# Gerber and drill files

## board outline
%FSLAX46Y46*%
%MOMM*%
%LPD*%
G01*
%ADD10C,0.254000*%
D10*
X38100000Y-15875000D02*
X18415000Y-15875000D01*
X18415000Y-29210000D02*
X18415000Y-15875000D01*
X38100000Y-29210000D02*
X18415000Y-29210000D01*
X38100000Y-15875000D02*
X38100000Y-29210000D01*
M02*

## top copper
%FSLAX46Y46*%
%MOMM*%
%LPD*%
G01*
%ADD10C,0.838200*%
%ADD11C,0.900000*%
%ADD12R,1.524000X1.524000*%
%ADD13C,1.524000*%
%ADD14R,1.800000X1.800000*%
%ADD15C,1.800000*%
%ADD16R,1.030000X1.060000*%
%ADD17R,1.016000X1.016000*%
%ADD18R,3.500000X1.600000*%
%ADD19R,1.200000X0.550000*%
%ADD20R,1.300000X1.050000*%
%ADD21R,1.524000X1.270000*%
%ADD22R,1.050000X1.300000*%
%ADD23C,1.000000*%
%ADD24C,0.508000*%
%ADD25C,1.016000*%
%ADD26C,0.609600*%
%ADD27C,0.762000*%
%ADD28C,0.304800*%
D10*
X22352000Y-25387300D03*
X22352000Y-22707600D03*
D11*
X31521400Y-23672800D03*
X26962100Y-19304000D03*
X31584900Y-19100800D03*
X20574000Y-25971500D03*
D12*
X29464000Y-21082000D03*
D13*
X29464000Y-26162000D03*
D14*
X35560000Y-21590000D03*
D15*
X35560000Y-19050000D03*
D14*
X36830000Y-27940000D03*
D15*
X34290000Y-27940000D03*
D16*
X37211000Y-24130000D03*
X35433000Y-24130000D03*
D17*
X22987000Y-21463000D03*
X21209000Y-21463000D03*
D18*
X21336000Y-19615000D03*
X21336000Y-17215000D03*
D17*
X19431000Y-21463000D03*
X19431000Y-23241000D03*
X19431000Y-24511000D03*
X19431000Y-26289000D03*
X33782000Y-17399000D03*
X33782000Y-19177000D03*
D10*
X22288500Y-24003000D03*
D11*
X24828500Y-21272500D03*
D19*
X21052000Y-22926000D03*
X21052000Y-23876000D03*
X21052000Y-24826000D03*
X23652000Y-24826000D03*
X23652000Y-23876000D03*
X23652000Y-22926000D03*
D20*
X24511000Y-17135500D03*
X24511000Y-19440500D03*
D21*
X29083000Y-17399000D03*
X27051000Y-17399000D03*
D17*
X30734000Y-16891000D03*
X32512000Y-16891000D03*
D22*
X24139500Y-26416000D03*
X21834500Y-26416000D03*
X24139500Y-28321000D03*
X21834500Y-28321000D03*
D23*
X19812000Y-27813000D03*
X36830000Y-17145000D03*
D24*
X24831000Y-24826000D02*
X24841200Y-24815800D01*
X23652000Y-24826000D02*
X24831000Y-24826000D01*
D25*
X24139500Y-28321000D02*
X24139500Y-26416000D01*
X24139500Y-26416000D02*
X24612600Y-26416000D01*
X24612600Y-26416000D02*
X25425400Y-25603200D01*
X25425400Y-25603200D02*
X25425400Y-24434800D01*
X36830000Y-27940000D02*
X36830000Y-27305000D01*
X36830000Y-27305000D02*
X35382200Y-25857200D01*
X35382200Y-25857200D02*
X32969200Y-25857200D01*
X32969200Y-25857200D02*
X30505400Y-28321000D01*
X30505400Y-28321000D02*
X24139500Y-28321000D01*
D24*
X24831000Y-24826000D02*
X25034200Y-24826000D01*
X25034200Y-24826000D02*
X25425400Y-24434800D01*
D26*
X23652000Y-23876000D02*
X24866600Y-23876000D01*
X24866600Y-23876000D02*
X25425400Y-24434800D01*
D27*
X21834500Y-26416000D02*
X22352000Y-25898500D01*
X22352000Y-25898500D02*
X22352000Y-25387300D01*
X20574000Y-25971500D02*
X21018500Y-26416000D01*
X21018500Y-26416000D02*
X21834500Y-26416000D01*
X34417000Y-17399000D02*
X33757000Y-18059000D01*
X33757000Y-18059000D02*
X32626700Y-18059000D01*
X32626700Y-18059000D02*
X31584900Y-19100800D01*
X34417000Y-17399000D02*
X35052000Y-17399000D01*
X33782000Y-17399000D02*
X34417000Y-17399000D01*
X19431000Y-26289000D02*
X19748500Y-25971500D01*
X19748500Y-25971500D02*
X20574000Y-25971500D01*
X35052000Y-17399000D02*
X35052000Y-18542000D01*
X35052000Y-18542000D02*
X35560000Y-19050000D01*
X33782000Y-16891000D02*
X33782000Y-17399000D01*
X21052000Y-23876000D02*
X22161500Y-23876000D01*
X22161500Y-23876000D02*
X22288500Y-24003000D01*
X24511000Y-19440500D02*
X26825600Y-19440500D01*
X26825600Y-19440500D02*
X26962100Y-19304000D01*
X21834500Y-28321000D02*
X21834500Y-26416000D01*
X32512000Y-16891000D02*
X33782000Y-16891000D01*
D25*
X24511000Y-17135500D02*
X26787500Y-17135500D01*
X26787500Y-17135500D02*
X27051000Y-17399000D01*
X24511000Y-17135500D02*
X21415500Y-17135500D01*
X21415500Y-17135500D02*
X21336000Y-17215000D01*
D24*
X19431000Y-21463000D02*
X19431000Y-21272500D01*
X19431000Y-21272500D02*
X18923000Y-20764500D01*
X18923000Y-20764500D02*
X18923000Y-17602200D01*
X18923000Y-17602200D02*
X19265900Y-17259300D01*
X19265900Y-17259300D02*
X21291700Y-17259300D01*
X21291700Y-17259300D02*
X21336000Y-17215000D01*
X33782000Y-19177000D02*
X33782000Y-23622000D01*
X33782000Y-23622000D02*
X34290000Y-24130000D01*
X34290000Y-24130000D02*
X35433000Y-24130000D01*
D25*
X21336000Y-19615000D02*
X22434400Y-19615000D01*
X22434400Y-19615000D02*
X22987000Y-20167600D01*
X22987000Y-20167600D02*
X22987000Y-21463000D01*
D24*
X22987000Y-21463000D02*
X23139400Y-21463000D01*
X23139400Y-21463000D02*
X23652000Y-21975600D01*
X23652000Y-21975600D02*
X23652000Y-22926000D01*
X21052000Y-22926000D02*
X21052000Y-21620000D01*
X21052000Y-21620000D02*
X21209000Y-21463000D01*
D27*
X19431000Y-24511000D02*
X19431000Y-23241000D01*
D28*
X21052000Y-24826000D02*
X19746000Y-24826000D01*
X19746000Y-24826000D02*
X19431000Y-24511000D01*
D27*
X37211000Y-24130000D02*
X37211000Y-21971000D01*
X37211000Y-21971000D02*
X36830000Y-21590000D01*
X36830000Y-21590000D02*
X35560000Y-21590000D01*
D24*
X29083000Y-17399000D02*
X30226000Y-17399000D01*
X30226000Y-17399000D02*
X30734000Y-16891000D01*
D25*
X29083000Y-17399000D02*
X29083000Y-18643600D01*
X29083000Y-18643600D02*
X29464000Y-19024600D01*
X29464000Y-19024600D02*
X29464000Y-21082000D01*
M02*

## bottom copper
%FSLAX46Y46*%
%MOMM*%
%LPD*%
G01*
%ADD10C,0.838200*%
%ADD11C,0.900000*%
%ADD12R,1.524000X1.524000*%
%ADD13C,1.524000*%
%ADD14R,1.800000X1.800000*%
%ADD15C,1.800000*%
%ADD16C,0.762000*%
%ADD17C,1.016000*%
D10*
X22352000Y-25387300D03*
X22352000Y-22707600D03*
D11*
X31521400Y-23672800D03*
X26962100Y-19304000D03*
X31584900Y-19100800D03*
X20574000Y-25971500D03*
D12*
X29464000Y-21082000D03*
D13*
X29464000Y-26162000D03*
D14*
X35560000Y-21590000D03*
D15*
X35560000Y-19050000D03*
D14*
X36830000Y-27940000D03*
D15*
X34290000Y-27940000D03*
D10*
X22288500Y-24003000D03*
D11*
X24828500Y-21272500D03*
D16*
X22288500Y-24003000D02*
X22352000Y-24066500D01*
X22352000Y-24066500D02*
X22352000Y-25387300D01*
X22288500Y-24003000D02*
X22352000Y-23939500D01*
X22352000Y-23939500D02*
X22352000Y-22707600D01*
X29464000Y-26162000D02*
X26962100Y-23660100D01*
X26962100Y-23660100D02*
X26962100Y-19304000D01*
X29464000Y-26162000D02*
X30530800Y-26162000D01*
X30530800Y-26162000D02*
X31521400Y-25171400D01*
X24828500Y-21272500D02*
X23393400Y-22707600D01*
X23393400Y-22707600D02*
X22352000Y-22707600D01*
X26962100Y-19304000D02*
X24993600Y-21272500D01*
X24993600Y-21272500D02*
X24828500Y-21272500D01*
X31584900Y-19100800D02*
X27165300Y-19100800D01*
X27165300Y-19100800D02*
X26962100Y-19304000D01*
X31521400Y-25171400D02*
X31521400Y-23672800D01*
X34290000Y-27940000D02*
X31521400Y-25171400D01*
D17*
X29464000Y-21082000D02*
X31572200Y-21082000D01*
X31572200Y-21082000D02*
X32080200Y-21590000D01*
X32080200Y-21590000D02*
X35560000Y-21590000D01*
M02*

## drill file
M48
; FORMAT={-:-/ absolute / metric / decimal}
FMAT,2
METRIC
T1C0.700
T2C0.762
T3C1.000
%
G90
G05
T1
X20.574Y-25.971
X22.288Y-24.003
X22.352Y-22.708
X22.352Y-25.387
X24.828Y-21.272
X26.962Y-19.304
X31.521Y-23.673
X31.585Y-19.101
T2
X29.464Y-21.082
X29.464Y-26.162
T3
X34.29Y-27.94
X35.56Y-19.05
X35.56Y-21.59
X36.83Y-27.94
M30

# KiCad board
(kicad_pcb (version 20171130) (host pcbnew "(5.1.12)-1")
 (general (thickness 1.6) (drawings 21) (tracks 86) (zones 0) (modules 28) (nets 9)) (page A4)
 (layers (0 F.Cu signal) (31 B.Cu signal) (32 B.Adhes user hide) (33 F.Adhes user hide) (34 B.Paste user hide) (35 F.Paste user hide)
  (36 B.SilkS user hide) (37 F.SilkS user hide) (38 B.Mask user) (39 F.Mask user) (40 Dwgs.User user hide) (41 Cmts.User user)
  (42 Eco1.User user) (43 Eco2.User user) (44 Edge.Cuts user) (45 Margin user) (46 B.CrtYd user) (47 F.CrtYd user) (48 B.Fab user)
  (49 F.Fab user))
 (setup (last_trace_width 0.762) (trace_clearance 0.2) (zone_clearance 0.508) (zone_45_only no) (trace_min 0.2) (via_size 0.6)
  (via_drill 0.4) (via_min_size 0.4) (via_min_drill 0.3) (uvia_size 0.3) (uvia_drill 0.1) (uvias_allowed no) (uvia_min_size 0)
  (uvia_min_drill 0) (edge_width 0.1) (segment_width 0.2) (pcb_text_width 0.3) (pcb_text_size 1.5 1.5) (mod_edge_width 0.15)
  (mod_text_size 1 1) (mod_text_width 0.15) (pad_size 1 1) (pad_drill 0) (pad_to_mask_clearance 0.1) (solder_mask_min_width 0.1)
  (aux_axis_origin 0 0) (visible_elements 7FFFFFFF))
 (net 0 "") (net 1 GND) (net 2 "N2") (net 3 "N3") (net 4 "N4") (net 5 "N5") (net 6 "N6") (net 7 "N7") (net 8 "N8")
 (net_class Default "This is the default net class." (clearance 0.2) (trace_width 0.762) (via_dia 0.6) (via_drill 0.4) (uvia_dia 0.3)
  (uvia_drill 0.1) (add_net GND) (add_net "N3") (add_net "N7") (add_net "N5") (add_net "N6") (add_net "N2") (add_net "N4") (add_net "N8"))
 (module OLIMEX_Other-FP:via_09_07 (layer F.Cu) (at 22.352 25.3873)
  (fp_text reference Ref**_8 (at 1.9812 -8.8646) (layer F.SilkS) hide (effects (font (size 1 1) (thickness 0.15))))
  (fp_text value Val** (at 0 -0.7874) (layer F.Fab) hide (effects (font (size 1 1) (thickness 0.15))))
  (pad 0 thru_hole circle (at 0 0) (size 0.8382 0.8382) (drill 0.7) (layers *.Cu) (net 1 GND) (zone_connect 2)))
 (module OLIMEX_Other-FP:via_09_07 (layer F.Cu) (at 22.352 22.7076)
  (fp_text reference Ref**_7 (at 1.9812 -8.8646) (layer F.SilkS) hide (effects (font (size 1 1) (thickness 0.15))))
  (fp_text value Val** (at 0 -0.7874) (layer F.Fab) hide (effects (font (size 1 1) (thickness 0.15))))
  (pad 0 thru_hole circle (at 0 0) (size 0.8382 0.8382) (drill 0.7) (layers *.Cu) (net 1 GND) (zone_connect 2)))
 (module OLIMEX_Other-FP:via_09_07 (layer F.Cu) (at 31.5214 23.7363)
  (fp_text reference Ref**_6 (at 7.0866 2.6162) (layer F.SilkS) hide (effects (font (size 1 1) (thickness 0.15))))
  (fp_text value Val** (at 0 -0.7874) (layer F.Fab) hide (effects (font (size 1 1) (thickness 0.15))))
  (pad 0 thru_hole circle (at 0 -0.0635) (size 0.9 0.9) (drill 0.7) (layers *.Cu) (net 1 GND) (zone_connect 2)))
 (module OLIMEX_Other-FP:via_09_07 (layer F.Cu) (at 26.9621 19.3675)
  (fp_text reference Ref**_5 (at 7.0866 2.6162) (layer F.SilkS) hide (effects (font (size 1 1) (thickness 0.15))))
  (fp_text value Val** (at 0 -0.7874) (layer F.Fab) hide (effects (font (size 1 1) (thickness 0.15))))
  (pad 0 thru_hole circle (at 0 -0.0635) (size 0.9 0.9) (drill 0.7) (layers *.Cu) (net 1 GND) (zone_connect 2)))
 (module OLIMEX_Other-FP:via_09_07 (layer F.Cu) (at 31.5849 19.1643)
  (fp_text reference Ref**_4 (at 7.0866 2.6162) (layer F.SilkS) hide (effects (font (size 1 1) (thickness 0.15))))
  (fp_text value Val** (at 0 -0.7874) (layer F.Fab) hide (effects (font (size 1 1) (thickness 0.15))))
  (pad 0 thru_hole circle (at 0 -0.0635) (size 0.9 0.9) (drill 0.7) (layers *.Cu) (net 1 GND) (zone_connect 2)))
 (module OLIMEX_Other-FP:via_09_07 (layer F.Cu) (at 20.574 26.035)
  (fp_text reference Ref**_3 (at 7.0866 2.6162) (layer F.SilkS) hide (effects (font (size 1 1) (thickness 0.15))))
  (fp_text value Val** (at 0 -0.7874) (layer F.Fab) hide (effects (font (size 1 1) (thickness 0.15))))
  (pad 0 thru_hole circle (at 0 -0.0635) (size 0.9 0.9) (drill 0.7) (layers *.Cu) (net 1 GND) (zone_connect 2)))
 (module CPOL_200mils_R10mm (layer F.Cu) (at 29.464 23.622 270)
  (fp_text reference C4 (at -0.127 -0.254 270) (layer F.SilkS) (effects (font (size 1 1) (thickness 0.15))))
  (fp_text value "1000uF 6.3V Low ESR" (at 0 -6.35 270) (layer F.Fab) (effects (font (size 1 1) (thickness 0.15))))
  (pad 1 thru_hole rect (at -2.54 0 270) (size 1.524 1.524) (drill 0.762) (layers *.Cu *.Mask F.SilkS) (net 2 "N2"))
  (pad 2 thru_hole circle (at 2.54 0 270) (size 1.524 1.524) (drill 0.762) (layers *.Cu *.Mask F.SilkS) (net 1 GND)))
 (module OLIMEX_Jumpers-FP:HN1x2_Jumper (layer F.Cu) (at 35.56 20.32 90)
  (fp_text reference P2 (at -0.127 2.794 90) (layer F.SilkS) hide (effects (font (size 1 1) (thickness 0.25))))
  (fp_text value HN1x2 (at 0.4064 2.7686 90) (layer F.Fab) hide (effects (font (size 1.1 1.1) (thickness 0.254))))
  (pad 1 thru_hole rect (at -1.27 0 180) (size 1.8 1.8) (drill 1) (layers *.Cu *.Mask F.SilkS) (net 2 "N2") (solder_mask_margin 0.0508)
   (solder_paste_margin -0.0508))
  (pad 2 thru_hole circle (at 1.27 0 180) (size 1.8 1.8) (drill 1) (layers *.Cu *.Mask F.SilkS) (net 1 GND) (solder_mask_margin 0.0508)
   (solder_paste_margin -0.0508)))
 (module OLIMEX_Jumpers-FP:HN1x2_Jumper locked (layer F.Cu) (at 35.56 27.94 180)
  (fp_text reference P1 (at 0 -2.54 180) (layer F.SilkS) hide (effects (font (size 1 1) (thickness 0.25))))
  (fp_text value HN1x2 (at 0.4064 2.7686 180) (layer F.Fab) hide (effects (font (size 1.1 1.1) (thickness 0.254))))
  (pad 1 thru_hole rect (at -1.27 0 270) (size 1.8 1.8) (drill 1) (layers *.Cu *.Mask F.SilkS) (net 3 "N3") (solder_mask_margin 0.0508)
   (solder_paste_margin -0.0508))
  (pad 2 thru_hole circle (at 1.27 0 270) (size 1.8 1.8) (drill 1) (layers *.Cu *.Mask F.SilkS) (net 1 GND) (solder_mask_margin 0.0508)
   (solder_paste_margin -0.0508)))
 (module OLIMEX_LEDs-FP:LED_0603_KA (layer F.Cu) (at 36.322 24.13 180)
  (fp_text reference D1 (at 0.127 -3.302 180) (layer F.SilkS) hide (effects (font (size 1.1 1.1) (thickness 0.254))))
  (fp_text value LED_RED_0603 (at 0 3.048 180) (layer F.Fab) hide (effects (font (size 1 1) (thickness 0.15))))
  (pad 2 smd rect (at -0.889 0 180) (size 1.03 1.06) (layers F.Cu F.Paste F.Mask) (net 2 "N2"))
  (pad 1 smd rect (at 0.889 0 180) (size 1.03 1.06) (layers F.Cu F.Paste F.Mask) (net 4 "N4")))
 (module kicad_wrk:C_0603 (layer F.Cu) (at 22.098 21.463 180)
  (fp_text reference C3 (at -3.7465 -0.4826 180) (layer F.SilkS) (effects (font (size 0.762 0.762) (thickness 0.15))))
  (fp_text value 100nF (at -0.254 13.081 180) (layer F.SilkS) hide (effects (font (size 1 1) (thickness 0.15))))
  (pad 1 smd rect (at -0.889 0 180) (size 1.016 1.016) (layers F.Cu F.Paste F.Mask) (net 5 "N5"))
  (pad 2 smd rect (at 0.889 0 180) (size 1.016 1.016) (layers F.Cu F.Paste F.Mask) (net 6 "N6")))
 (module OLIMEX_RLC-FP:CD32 (layer F.Cu) (at 21.336 18.415 90)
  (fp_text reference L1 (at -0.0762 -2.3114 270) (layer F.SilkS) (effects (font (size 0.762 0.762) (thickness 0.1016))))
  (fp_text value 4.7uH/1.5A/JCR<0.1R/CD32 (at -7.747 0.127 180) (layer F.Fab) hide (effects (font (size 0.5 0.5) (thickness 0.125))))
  (pad 1 smd rect (at -1.2 0 180) (size 3.5 1.6) (layers F.Cu F.Paste F.Mask) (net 5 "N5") (solder_mask_margin 0.0508)
   (solder_paste_margin -0.0508) (clearance 0.0508))
  (pad 2 smd rect (at 1.2 0 180) (size 3.5 1.6) (layers F.Cu F.Paste F.Mask) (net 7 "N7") (solder_mask_margin 0.0508)
   (solder_paste_margin -0.0508) (clearance 0.0508)))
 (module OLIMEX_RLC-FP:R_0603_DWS (layer F.Cu) (at 19.431 22.352 270)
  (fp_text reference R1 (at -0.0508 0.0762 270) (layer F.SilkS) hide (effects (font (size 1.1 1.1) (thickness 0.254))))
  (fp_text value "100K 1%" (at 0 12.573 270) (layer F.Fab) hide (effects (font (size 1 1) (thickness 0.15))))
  (pad 1 smd rect (at -0.889 0 270) (size 1.016 1.016) (layers F.Cu F.Paste F.Mask) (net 7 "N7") (solder_mask_margin 0.0508)
   (solder_paste_margin -0.0508) (clearance 0.0508))
  (pad 2 smd rect (at 0.889 0 270) (size 1.016 1.016) (layers F.Cu F.Paste F.Mask) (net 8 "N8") (solder_mask_margin 0.0508)
   (solder_paste_margin -0.0508) (clearance 0.0508)))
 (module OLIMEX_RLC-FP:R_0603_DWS (layer F.Cu) (at 19.431 25.4 270)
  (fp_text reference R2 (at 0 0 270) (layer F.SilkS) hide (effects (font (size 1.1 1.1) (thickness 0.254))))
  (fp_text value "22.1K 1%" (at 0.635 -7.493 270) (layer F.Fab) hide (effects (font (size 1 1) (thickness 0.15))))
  (pad 1 smd rect (at -0.889 0 270) (size 1.016 1.016) (layers F.Cu F.Paste F.Mask) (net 8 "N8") (solder_mask_margin 0.0508)
   (solder_paste_margin -0.0508) (clearance 0.0508))
  (pad 2 smd rect (at 0.889 0 270) (size 1.016 1.016) (layers F.Cu F.Paste F.Mask) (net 1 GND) (solder_mask_margin 0.0508)
   (solder_paste_margin -0.0508) (clearance 0.0508)))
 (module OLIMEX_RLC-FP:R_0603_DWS (layer F.Cu) (at 33.782 18.288 270)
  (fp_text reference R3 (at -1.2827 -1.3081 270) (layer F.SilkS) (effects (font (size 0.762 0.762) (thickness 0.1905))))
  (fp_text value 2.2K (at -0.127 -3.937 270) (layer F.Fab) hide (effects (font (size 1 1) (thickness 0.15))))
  (pad 1 smd rect (at -0.889 0 270) (size 1.016 1.016) (layers F.Cu F.Paste F.Mask) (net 1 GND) (solder_mask_margin 0.0508)
   (solder_paste_margin -0.0508) (clearance 0.0508))
  (pad 2 smd rect (at 0.889 0 270) (size 1.016 1.016) (layers F.Cu F.Paste F.Mask) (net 4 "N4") (solder_mask_margin 0.0508)
   (solder_paste_margin -0.0508) (clearance 0.0508)))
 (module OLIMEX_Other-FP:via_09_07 (layer F.Cu) (at 22.2885 24.003)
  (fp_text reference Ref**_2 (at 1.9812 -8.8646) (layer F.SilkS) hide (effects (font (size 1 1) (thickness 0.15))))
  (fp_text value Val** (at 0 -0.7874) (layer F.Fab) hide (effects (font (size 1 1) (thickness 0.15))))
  (pad 0 thru_hole circle (at 0 0) (size 0.8382 0.8382) (drill 0.7) (layers *.Cu) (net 1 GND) (zone_connect 2)))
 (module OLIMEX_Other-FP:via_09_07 (layer F.Cu) (at 24.8285 21.336)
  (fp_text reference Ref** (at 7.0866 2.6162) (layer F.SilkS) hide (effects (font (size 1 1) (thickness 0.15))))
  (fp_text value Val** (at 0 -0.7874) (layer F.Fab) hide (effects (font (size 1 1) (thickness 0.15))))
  (pad 0 thru_hole circle (at 0 -0.0635) (size 0.9 0.9) (drill 0.7) (layers *.Cu) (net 1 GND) (zone_connect 2)))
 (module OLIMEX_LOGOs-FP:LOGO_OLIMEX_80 (layer B.Cu) (at 27.6606 23.0378 180)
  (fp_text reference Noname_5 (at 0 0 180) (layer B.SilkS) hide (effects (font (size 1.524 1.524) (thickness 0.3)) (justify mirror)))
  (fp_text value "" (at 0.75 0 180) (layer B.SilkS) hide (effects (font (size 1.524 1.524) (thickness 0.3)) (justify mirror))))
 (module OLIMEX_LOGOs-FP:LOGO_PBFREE (layer B.Cu) (at 26.5938 18.796 180)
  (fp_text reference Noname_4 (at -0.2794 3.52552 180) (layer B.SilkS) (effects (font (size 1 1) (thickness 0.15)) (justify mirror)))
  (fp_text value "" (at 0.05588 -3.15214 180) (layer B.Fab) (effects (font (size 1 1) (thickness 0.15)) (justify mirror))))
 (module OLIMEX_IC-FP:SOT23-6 (layer F.Cu) (at 22.352 23.876 180)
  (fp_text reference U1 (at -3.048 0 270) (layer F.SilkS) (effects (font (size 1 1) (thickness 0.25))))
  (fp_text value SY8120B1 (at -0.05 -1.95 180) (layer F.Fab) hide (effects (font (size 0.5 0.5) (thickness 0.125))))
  (pad 1 smd rect (at 1.3 0.95 270) (size 0.55 1.2) (layers F.Cu F.Paste F.Mask) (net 6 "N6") (solder_mask_margin 0.0508)
   (solder_paste_margin -0.0508) (clearance 0.0508))
  (pad 2 smd rect (at 1.3 0 270) (size 0.55 1.2) (layers F.Cu F.Paste F.Mask) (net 1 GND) (solder_mask_margin 0.0508)
   (solder_paste_margin -0.0508) (clearance 0.0508))
  (pad 3 smd rect (at 1.3 -0.95 270) (size 0.55 1.2) (layers F.Cu F.Paste F.Mask) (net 8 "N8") (solder_mask_margin 0.0508)
   (solder_paste_margin -0.0508) (clearance 0.0508))
  (pad 4 smd rect (at -1.3 -0.95 270) (size 0.55 1.2) (layers F.Cu F.Paste F.Mask) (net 3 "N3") (solder_mask_margin 0.0508)
   (solder_paste_margin -0.0508) (clearance 0.0508))
  (pad 5 smd rect (at -1.3 0 270) (size 0.55 1.2) (layers F.Cu F.Paste F.Mask) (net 3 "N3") (solder_mask_margin 0.0508)
   (solder_paste_margin -0.0508) (clearance 0.0508))
  (pad 6 smd rect (at -1.3 0.95 270) (size 0.55 1.2) (layers F.Cu F.Paste F.Mask) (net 5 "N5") (solder_mask_margin 0.0508)
   (solder_paste_margin -0.0508) (clearance 0.0508)))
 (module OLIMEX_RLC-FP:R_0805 (layer F.Cu) (at 24.511 18.288)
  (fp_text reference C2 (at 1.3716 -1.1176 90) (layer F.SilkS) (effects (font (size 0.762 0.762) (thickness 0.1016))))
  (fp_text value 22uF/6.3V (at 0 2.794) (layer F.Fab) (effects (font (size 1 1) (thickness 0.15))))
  (pad 1 smd rect (at 0 -1.1525) (size 1.3 1.05) (layers F.Cu F.Paste F.Mask) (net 7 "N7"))
  (pad 2 smd rect (at 0 1.1525) (size 1.3 1.05) (layers F.Cu F.Paste F.Mask) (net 1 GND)))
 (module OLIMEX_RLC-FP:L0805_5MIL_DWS (layer F.Cu) (at 28.067 17.399)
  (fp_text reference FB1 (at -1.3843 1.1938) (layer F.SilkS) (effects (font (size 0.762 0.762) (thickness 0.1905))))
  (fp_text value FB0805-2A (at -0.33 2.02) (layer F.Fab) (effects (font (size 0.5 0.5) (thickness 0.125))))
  (pad 2 smd rect (at 1.016 0) (size 1.524 1.27) (layers F.Cu F.Paste F.Mask) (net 2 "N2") (solder_mask_margin 0.0508)
   (solder_paste_margin -0.0508) (clearance 0.0508))
  (pad 1 smd rect (at -1.016 0) (size 1.524 1.27) (layers F.Cu F.Paste F.Mask) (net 7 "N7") (solder_mask_margin 0.0508)
   (solder_paste_margin -0.0508) (clearance 0.0508)))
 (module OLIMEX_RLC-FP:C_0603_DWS (layer F.Cu) (at 31.623 16.891)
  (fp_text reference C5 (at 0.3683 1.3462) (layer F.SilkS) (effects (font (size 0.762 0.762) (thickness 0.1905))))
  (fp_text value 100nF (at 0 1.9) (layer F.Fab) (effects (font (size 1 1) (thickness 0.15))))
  (pad 1 smd rect (at -0.889 0) (size 1.016 1.016) (layers F.Cu F.Paste F.Mask) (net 2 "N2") (solder_mask_margin 0.0508)
   (solder_paste_margin -0.0508) (clearance 0.0508))
  (pad 2 smd rect (at 0.889 0) (size 1.016 1.016) (layers F.Cu F.Paste F.Mask) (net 1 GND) (solder_mask_margin 0.0508)
   (solder_paste_margin -0.0508) (clearance 0.0508)))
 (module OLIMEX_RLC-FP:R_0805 (layer F.Cu) (at 22.987 26.416 270)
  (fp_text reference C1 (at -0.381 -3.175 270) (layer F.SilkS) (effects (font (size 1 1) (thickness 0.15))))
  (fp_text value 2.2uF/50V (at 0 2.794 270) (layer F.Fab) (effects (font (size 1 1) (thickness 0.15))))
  (pad 1 smd rect (at 0 -1.1525 270) (size 1.3 1.05) (layers F.Cu F.Paste F.Mask) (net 3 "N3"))
  (pad 2 smd rect (at 0 1.1525 270) (size 1.3 1.05) (layers F.Cu F.Paste F.Mask) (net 1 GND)))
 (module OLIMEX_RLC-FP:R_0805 (layer F.Cu) (at 22.987 28.321 270)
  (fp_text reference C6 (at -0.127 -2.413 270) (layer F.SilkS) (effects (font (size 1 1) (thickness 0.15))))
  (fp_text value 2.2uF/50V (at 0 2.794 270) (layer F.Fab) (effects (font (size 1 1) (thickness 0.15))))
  (pad 1 smd rect (at 0 -1.1525 270) (size 1.3 1.05) (layers F.Cu F.Paste F.Mask) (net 3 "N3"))
  (pad 2 smd rect (at 0 1.1525 270) (size 1.3 1.05) (layers F.Cu F.Paste F.Mask) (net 1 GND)))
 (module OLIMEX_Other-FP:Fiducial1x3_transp (layer F.Cu) (at 19.812 27.813)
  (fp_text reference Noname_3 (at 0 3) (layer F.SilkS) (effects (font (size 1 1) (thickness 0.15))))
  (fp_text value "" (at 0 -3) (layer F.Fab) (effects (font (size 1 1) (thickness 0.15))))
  (pad Fid1 connect circle (at 0 0) (size 1 1) (layers F.Cu F.Mask) (clearance 0.4) (zone_connect 0)))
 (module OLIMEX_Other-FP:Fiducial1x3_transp (layer F.Cu) (at 36.83 17.145)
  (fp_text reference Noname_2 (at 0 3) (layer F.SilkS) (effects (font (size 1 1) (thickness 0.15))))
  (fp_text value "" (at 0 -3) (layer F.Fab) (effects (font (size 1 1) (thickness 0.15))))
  (pad Fid1 connect circle (at 0 0) (size 1 1) (layers F.Cu F.Mask) (clearance 0.6) (zone_connect 0)))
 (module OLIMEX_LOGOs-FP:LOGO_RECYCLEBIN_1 (layer B.Cu) (at 23.8379 22.3266 180)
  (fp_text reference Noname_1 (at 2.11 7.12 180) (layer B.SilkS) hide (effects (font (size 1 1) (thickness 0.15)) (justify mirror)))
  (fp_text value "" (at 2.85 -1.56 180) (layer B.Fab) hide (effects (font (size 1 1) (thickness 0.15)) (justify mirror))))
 (gr_line (start 38.1 15.875) (end 18.415 15.875) (angle 90) (layer Edge.Cuts) (width 0.254))
 (gr_line (start 18.415 29.21) (end 18.415 15.875) (angle 90) (layer Edge.Cuts) (width 0.254))
 (gr_line (start 38.1 29.21) (end 18.415 29.21) (angle 90) (layer Edge.Cuts) (width 0.254))
 (gr_line (start 38.1 15.875) (end 38.1 29.21) (angle 90) (layer Edge.Cuts) (width 0.254))
 (segment (start 24.831 24.826) (end 24.8412 24.8158) (width 0.508) (layer F.Cu) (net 3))
 (segment (start 23.652 24.826) (end 24.831 24.826) (width 0.508) (layer F.Cu) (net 3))
 (segment (start 24.1395 28.321) (end 24.1395 26.416) (width 1.016) (layer F.Cu) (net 3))
 (segment (start 24.1395 26.416) (end 24.6126 26.416) (width 1.016) (layer F.Cu) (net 3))
 (segment (start 24.6126 26.416) (end 25.4254 25.6032) (width 1.016) (layer F.Cu) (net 3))
 (segment (start 25.4254 25.6032) (end 25.4254 24.4348) (width 1.016) (layer F.Cu) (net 3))
 (segment (start 36.83 27.94) (end 36.83 27.305) (width 1.016) (layer F.Cu) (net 3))
 (segment (start 36.83 27.305) (end 35.3822 25.8572) (width 1.016) (layer F.Cu) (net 3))
 (segment (start 35.3822 25.8572) (end 32.9692 25.8572) (width 1.016) (layer F.Cu) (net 3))
 (segment (start 32.9692 25.8572) (end 30.5054 28.321) (width 1.016) (layer F.Cu) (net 3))
 (segment (start 30.5054 28.321) (end 24.1395 28.321) (width 1.016) (layer F.Cu) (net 3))
 (segment (start 24.831 24.826) (end 25.0342 24.826) (width 0.508) (layer F.Cu) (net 3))
 (segment (start 25.0342 24.826) (end 25.4254 24.4348) (width 0.508) (layer F.Cu) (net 3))
 (segment (start 23.652 23.876) (end 24.8666 23.876) (width 0.6096) (layer F.Cu) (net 3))
 (segment (start 24.8666 23.876) (end 25.4254 24.4348) (width 0.6096) (layer F.Cu) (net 3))
 (segment (start 22.2885 24.003) (end 22.352 24.0665) (width 0.762) (layer B.Cu) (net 1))
 (segment (start 22.352 24.0665) (end 22.352 25.3873) (width 0.762) (layer B.Cu) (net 1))
 (segment (start 22.2885 24.003) (end 22.352 23.9395) (width 0.762) (layer B.Cu) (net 1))
 (segment (start 22.352 23.9395) (end 22.352 22.7076) (width 0.762) (layer B.Cu) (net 1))
 (segment (start 29.464 26.162) (end 26.9621 23.6601) (width 0.762) (layer B.Cu) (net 1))
 (segment (start 26.9621 23.6601) (end 26.9621 19.304) (width 0.762) (layer B.Cu) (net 1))
 (segment (start 29.464 26.162) (end 30.5308 26.162) (width 0.762) (layer B.Cu) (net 1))
 (segment (start 30.5308 26.162) (end 31.5214 25.1714) (width 0.762) (layer B.Cu) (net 1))
 (segment (start 24.8285 21.2725) (end 23.3934 22.7076) (width 0.762) (layer B.Cu) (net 1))
 (segment (start 23.3934 22.7076) (end 22.352 22.7076) (width 0.762) (layer B.Cu) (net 1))
 (segment (start 26.9621 19.304) (end 24.9936 21.2725) (width 0.762) (layer B.Cu) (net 1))
 (segment (start 24.9936 21.2725) (end 24.8285 21.2725) (width 0.762) (layer B.Cu) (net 1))
 (segment (start 31.5849 19.1008) (end 27.1653 19.1008) (width 0.762) (layer B.Cu) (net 1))
 (segment (start 27.1653 19.1008) (end 26.9621 19.304) (width 0.762) (layer B.Cu) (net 1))
 (segment (start 21.8345 26.416) (end 22.352 25.8985) (width 0.762) (layer F.Cu) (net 1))
 (segment (start 22.352 25.8985) (end 22.352 25.3873) (width 0.762) (layer F.Cu) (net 1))
 (segment (start 20.574 25.9715) (end 21.0185 26.416) (width 0.762) (layer F.Cu) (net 1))
 (segment (start 21.0185 26.416) (end 21.8345 26.416) (width 0.762) (layer F.Cu) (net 1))
 (segment (start 31.5214 25.1714) (end 31.5214 23.6728) (width 0.762) (layer B.Cu) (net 1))
 (segment (start 34.29 27.94) (end 31.5214 25.1714) (width 0.762) (layer B.Cu) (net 1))
 (segment (start 34.417 17.399) (end 33.757 18.059) (width 0.762) (layer F.Cu) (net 1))
 (segment (start 33.757 18.059) (end 32.6267 18.059) (width 0.762) (layer F.Cu) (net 1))
 (segment (start 32.6267 18.059) (end 31.5849 19.1008) (width 0.762) (layer F.Cu) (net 1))
 (segment (start 34.417 17.399) (end 35.052 17.399) (width 0.762) (layer F.Cu) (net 1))
 (segment (start 33.782 17.399) (end 34.417 17.399) (width 0.762) (layer F.Cu) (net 1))
 (segment (start 19.431 26.289) (end 19.7485 25.9715) (width 0.762) (layer F.Cu) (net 1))
 (segment (start 19.7485 25.9715) (end 20.574 25.9715) (width 0.762) (layer F.Cu) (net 1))
 (segment (start 35.052 17.399) (end 35.052 18.542) (width 0.762) (layer F.Cu) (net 1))
 (segment (start 35.052 18.542) (end 35.56 19.05) (width 0.762) (layer F.Cu) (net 1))
 (segment (start 33.782 16.891) (end 33.782 17.399) (width 0.762) (layer F.Cu) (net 1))
 (segment (start 21.052 23.876) (end 22.1615 23.876) (width 0.762) (layer F.Cu) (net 1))
 (segment (start 22.1615 23.876) (end 22.2885 24.003) (width 0.762) (layer F.Cu) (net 1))
 (segment (start 24.511 19.4405) (end 26.8256 19.4405) (width 0.762) (layer F.Cu) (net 1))
 (segment (start 26.8256 19.4405) (end 26.9621 19.304) (width 0.762) (layer F.Cu) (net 1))
 (segment (start 21.8345 28.321) (end 21.8345 26.416) (width 0.762) (layer F.Cu) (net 1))
 (segment (start 32.512 16.891) (end 33.782 16.891) (width 0.762) (layer F.Cu) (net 1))
 (segment (start 24.511 17.1355) (end 26.7875 17.1355) (width 1.016) (layer F.Cu) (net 7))
 (segment (start 26.7875 17.1355) (end 27.051 17.399) (width 1.016) (layer F.Cu) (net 7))
 (segment (start 24.511 17.1355) (end 21.4155 17.1355) (width 1.016) (layer F.Cu) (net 7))
 (segment (start 21.4155 17.1355) (end 21.336 17.215) (width 1.016) (layer F.Cu) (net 7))
 (segment (start 19.431 21.463) (end 19.431 21.2725) (width 0.508) (layer F.Cu) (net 7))
 (segment (start 19.431 21.2725) (end 18.923 20.7645) (width 0.508) (layer F.Cu) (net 7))
 (segment (start 18.923 20.7645) (end 18.923 17.6022) (width 0.508) (layer F.Cu) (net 7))
 (segment (start 18.923 17.6022) (end 19.2659 17.2593) (width 0.508) (layer F.Cu) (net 7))
 (segment (start 19.2659 17.2593) (end 21.2917 17.2593) (width 0.508) (layer F.Cu) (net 7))
 (segment (start 21.2917 17.2593) (end 21.336 17.215) (width 0.508) (layer F.Cu) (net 7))
 (segment (start 33.782 19.177) (end 33.782 23.622) (width 0.508) (layer F.Cu) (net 4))
 (segment (start 33.782 23.622) (end 34.29 24.13) (width 0.508) (layer F.Cu) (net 4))
 (segment (start 34.29 24.13) (end 35.433 24.13) (width 0.508) (layer F.Cu) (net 4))
 (segment (start 21.336 19.615) (end 22.4344 19.615) (width 1.016) (layer F.Cu) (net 5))
 (segment (start 22.4344 19.615) (end 22.987 20.1676) (width 1.016) (layer F.Cu) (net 5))
 (segment (start 22.987 20.1676) (end 22.987 21.463) (width 1.016) (layer F.Cu) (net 5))
 (segment (start 22.987 21.463) (end 23.1394 21.463) (width 0.508) (layer F.Cu) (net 5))
 (segment (start 23.1394 21.463) (end 23.652 21.9756) (width 0.508) (layer F.Cu) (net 5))
 (segment (start 23.652 21.9756) (end 23.652 22.926) (width 0.508) (layer F.Cu) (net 5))
 (segment (start 21.052 22.926) (end 21.052 21.62) (width 0.508) (layer F.Cu) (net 6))
 (segment (start 21.052 21.62) (end 21.209 21.463) (width 0.508) (layer F.Cu) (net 6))
 (segment (start 19.431 24.511) (end 19.431 23.241) (width 0.762) (layer F.Cu) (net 8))
 (segment (start 21.052 24.826) (end 19.746 24.826) (width 0.3048) (layer F.Cu) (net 8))
 (segment (start 19.746 24.826) (end 19.431 24.511) (width 0.3048) (layer F.Cu) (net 8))
 (segment (start 37.211 24.13) (end 37.211 21.971) (width 0.762) (layer F.Cu) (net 2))
 (segment (start 37.211 21.971) (end 36.83 21.59) (width 0.762) (layer F.Cu) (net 2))
 (segment (start 36.83 21.59) (end 35.56 21.59) (width 0.762) (layer F.Cu) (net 2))
 (segment (start 29.083 17.399) (end 30.226 17.399) (width 0.508) (layer F.Cu) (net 2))
 (segment (start 30.226 17.399) (end 30.734 16.891) (width 0.508) (layer F.Cu) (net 2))
 (segment (start 29.083 17.399) (end 29.083 18.6436) (width 1.016) (layer F.Cu) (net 2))
 (segment (start 29.083 18.6436) (end 29.464 19.0246) (width 1.016) (layer F.Cu) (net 2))
 (segment (start 29.464 19.0246) (end 29.464 21.082) (width 1.016) (layer F.Cu) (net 2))
 (segment (start 29.464 21.082) (end 31.5722 21.082) (width 1.016) (layer B.Cu) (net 2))
 (segment (start 31.5722 21.082) (end 32.0802 21.59) (width 1.016) (layer B.Cu) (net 2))
 (segment (start 32.0802 21.59) (end 35.56 21.59) (width 1.016) (layer B.Cu) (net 2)))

